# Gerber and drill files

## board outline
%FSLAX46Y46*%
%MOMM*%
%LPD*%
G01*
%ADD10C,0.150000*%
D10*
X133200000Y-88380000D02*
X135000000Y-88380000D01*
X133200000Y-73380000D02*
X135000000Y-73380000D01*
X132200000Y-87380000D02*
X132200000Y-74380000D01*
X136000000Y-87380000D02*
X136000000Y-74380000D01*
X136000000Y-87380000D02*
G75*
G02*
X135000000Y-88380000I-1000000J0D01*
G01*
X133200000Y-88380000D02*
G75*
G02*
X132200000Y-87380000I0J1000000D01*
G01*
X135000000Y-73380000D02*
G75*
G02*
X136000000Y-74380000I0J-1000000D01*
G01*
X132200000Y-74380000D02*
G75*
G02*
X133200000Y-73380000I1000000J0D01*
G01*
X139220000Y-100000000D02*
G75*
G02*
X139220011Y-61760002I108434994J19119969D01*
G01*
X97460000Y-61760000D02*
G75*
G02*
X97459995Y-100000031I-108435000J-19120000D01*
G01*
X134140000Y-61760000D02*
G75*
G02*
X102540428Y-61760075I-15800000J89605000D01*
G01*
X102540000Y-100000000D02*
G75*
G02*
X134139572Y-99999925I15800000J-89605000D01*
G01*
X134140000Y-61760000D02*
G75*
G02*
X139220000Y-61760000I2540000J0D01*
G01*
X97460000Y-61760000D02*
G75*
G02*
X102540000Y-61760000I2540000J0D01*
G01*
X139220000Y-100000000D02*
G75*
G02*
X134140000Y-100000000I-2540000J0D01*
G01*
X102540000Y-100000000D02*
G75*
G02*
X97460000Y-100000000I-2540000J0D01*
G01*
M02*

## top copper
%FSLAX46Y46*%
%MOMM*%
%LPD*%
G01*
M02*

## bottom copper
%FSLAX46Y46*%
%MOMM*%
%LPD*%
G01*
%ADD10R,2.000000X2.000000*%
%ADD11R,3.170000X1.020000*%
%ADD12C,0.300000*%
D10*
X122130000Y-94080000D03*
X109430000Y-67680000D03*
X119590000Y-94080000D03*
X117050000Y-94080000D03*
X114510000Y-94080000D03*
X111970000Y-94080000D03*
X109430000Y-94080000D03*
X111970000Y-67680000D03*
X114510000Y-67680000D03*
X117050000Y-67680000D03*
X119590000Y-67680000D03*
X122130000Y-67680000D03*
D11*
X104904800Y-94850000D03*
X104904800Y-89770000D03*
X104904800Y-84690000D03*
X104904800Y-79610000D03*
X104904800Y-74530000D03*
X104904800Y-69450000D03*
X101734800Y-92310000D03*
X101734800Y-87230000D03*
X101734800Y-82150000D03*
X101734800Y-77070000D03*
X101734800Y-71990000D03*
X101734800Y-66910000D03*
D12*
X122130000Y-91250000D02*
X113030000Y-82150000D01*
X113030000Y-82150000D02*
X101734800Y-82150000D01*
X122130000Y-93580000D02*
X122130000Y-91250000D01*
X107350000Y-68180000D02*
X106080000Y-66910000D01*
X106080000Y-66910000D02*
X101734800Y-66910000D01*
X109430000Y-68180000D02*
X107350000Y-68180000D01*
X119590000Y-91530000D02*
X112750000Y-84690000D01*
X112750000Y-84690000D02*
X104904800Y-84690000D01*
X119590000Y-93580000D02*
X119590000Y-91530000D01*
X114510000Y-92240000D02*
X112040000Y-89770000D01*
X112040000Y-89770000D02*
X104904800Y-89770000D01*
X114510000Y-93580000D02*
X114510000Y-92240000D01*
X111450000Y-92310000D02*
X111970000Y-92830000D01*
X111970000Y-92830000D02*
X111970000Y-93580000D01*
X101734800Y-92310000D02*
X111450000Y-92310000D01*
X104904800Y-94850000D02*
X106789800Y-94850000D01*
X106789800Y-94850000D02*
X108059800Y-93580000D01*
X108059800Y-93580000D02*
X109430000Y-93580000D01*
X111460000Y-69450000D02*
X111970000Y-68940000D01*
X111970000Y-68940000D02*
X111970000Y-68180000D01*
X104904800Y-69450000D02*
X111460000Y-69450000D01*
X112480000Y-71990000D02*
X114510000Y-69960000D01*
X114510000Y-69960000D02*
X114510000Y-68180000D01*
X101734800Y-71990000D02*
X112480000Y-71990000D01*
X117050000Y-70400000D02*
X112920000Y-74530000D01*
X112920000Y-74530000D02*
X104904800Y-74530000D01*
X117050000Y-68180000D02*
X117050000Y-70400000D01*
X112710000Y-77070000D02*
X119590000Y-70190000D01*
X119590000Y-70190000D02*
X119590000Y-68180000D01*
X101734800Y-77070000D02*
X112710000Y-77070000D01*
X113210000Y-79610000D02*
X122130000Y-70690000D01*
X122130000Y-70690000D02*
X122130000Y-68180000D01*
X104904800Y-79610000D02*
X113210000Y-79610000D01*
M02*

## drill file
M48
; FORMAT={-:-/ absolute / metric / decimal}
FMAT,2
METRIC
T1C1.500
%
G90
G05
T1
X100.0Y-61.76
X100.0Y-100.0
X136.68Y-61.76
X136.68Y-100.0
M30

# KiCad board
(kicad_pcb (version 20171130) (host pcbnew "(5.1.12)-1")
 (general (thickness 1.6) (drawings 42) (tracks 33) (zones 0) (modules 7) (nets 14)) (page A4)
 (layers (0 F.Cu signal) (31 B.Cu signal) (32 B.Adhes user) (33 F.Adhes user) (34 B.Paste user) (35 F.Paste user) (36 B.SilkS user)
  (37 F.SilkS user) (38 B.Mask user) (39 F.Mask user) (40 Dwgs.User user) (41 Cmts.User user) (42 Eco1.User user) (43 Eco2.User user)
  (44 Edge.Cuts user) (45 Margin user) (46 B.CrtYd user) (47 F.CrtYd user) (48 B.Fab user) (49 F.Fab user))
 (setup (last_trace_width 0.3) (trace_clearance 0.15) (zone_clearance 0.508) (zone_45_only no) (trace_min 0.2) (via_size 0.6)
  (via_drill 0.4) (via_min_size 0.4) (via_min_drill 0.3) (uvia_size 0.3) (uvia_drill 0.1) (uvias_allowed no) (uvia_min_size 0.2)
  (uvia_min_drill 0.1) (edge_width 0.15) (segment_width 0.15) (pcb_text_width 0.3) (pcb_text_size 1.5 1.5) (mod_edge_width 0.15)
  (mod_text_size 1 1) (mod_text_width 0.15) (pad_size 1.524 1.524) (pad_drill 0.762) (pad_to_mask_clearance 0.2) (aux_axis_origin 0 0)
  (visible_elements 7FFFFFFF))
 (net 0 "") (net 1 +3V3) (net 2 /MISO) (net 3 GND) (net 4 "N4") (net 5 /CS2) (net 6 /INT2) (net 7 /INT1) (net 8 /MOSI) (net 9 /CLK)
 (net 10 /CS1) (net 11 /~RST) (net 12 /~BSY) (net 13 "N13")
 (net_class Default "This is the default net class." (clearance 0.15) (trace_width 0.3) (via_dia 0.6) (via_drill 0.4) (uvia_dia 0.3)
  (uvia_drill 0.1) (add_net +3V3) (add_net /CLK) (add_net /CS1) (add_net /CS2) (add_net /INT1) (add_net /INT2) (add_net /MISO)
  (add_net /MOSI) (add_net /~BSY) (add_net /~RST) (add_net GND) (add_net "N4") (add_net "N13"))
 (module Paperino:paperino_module (layer B.Cu) (at 118.73 80.88 90)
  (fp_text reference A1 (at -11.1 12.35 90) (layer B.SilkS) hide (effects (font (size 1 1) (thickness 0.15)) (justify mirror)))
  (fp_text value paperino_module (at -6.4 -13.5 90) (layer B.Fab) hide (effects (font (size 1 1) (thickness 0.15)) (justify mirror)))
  (pad 1 smd rect (at -12.7 3.4 90) (size 2 2) (drill (offset -0.5 0)) (layers B.Cu B.Paste B.Mask) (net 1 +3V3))
  (pad 7 smd rect (at 12.7 -9.3 90) (size 2 2) (drill (offset 0.5 0)) (layers B.Cu B.Paste B.Mask) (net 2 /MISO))
  (pad 2 smd rect (at -12.7 0.86 90) (size 2 2) (drill (offset -0.5 0)) (layers B.Cu B.Paste B.Mask) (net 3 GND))
  (pad 3 smd rect (at -12.7 -1.68 90) (size 2 2) (drill (offset -0.5 0)) (layers B.Cu B.Paste B.Mask) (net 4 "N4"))
  (pad 4 smd rect (at -12.7 -4.22 90) (size 2 2) (drill (offset -0.5 0)) (layers B.Cu B.Paste B.Mask) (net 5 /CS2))
  (pad 5 smd rect (at -12.7 -6.76 90) (size 2 2) (drill (offset -0.5 0)) (layers B.Cu B.Paste B.Mask) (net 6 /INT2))
  (pad 6 smd rect (at -12.7 -9.3 90) (size 2 2) (drill (offset -0.5 0)) (layers B.Cu B.Paste B.Mask) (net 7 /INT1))
  (pad 8 smd rect (at 12.7 -6.76 90) (size 2 2) (drill (offset 0.5 0)) (layers B.Cu B.Paste B.Mask) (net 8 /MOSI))
  (pad 9 smd rect (at 12.7 -4.22 90) (size 2 2) (drill (offset 0.5 0)) (layers B.Cu B.Paste B.Mask) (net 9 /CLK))
  (pad 10 smd rect (at 12.7 -1.68 90) (size 2 2) (drill (offset 0.5 0)) (layers B.Cu B.Paste B.Mask) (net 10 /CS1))
  (pad 11 smd rect (at 12.7 0.86 90) (size 2 2) (drill (offset 0.5 0)) (layers B.Cu B.Paste B.Mask) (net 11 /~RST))
  (pad 12 smd rect (at 12.7 3.4 90) (size 2 2) (drill (offset 0.5 0)) (layers B.Cu B.Paste B.Mask) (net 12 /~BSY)))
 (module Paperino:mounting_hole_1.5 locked (layer F.Cu) (at 100 100)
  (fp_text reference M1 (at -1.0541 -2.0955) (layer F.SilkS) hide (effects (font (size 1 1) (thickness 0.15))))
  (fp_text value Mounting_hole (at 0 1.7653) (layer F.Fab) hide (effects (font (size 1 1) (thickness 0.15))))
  (pad "" np_thru_hole circle (at 0 0) (size 1.5 1.5) (drill 1.5) (layers *.Cu *.Mask)))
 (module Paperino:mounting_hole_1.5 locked (layer F.Cu) (at 136.68 100)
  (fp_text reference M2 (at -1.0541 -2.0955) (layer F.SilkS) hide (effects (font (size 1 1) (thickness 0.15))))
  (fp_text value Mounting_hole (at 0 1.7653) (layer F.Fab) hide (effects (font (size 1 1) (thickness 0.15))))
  (pad "" np_thru_hole circle (at 0 0) (size 1.5 1.5) (drill 1.5) (layers *.Cu *.Mask)))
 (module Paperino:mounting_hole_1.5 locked (layer F.Cu) (at 100 61.76)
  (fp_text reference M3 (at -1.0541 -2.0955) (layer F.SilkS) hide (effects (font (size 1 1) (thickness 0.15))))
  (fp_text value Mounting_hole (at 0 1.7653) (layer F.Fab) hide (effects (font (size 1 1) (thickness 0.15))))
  (pad "" np_thru_hole circle (at 0 0) (size 1.5 1.5) (drill 1.5) (layers *.Cu *.Mask)))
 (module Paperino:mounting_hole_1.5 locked (layer F.Cu) (at 136.68 61.76)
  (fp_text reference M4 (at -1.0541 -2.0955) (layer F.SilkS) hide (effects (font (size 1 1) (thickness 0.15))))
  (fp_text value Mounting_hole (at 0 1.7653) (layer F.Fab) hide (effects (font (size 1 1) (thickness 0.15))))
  (pad "" np_thru_hole circle (at 0 0) (size 1.5 1.5) (drill 1.5) (layers *.Cu *.Mask)))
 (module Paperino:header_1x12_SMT (layer B.Cu) (at 103.32 80.88 90)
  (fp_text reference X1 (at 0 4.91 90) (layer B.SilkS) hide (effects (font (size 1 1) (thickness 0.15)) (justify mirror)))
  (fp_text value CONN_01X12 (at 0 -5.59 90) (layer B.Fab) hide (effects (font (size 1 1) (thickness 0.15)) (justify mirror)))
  (pad 1 smd rect (at -13.97 1.5848 90) (size 1.02 3.17) (layers B.Cu B.Paste B.Mask) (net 7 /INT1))
  (pad 3 smd rect (at -8.89 1.5848 90) (size 1.02 3.17) (layers B.Cu B.Paste B.Mask) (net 5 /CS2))
  (pad 5 smd rect (at -3.81 1.5848 90) (size 1.02 3.17) (layers B.Cu B.Paste B.Mask) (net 3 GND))
  (pad 7 smd rect (at 1.27 1.5848 90) (size 1.02 3.17) (layers B.Cu B.Paste B.Mask) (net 12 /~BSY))
  (pad 9 smd rect (at 6.35 1.5848 90) (size 1.02 3.17) (layers B.Cu B.Paste B.Mask) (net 10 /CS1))
  (pad 11 smd rect (at 11.43 1.5848 90) (size 1.02 3.17) (layers B.Cu B.Paste B.Mask) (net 8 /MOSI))
  (pad 2 smd rect (at -11.43 -1.5852 90) (size 1.02 3.17) (layers B.Cu B.Paste B.Mask) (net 6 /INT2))
  (pad 4 smd rect (at -6.35 -1.5852 90) (size 1.02 3.17) (layers B.Cu B.Paste B.Mask) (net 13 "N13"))
  (pad 6 smd rect (at -1.27 -1.5852 90) (size 1.02 3.17) (layers B.Cu B.Paste B.Mask) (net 1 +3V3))
  (pad 8 smd rect (at 3.81 -1.5852 90) (size 1.02 3.17) (layers B.Cu B.Paste B.Mask) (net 11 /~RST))
  (pad 10 smd rect (at 8.89 -1.5852 90) (size 1.02 3.17) (layers B.Cu B.Paste B.Mask) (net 9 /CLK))
  (pad 12 smd rect (at 13.97 -1.5852 90) (size 1.02 3.17) (layers B.Cu B.Paste B.Mask) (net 2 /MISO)))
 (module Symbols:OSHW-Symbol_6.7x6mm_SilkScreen (layer F.Cu) (at 133.66 67.9 90)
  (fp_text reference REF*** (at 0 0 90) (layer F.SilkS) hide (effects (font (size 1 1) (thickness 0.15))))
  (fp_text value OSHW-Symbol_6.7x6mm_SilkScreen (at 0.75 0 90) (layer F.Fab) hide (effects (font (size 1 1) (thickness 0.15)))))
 (gr_line (start 133.2 88.38) (end 135 88.38) (layer Edge.Cuts) (width 0.15))
 (gr_line (start 133.2 73.38) (end 135 73.38) (layer Edge.Cuts) (width 0.15))
 (gr_line (start 132.2 87.38) (end 132.2 74.38) (layer Edge.Cuts) (width 0.15))
 (gr_line (start 136 87.38) (end 136 74.38) (layer Edge.Cuts) (width 0.15))
 (gr_arc (start 135 87.38) (end 136 87.38) (angle 90) (layer Edge.Cuts) (width 0.15))
 (gr_arc (start 133.2 87.38) (end 133.2 88.38) (angle 90) (layer Edge.Cuts) (width 0.15))
 (gr_arc (start 135 74.38) (end 135 73.38) (angle 90) (layer Edge.Cuts) (width 0.15))
 (gr_arc (start 133.2 74.38) (end 132.2 74.38) (angle 90) (layer Edge.Cuts) (width 0.15))
 (gr_arc (start 247.654994 80.880031) (end 139.22 100) (angle 19.9999845) (layer Edge.Cuts) (width 0.15))
 (gr_arc (start -10.975 80.88) (end 97.46 61.76) (angle 20) (layer Edge.Cuts) (width 0.15))
 (gr_arc (start 118.34 -27.845) (end 134.14 61.76) (angle 20) (layer Edge.Cuts) (width 0.15))
 (gr_arc (start 118.34 189.605) (end 102.54 100) (angle 20) (layer Edge.Cuts) (width 0.15))
 (gr_arc (start 136.68 61.76) (end 134.14 61.76) (angle 180) (layer Edge.Cuts) (width 0.15))
 (gr_arc (start 100 61.76) (end 97.46 61.76) (angle 180) (layer Edge.Cuts) (width 0.15))
 (gr_arc (start 136.68 100) (end 139.22 100) (angle 180) (layer Edge.Cuts) (width 0.15))
 (gr_arc (start 100 100) (end 102.54 100) (angle 180) (layer Edge.Cuts) (width 0.15))
 (segment (start 122.13 91.25) (end 113.03 82.15) (width 0.3) (layer B.Cu) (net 1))
 (segment (start 113.03 82.15) (end 101.7348 82.15) (width 0.3) (layer B.Cu) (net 1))
 (segment (start 122.13 93.58) (end 122.13 91.25) (width 0.3) (layer B.Cu) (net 1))
 (segment (start 107.35 68.18) (end 106.08 66.91) (width 0.3) (layer B.Cu) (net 2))
 (segment (start 106.08 66.91) (end 101.7348 66.91) (width 0.3) (layer B.Cu) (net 2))
 (segment (start 109.43 68.18) (end 107.35 68.18) (width 0.3) (layer B.Cu) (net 2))
 (segment (start 119.59 91.53) (end 112.75 84.69) (width 0.3) (layer B.Cu) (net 3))
 (segment (start 112.75 84.69) (end 104.9048 84.69) (width 0.3) (layer B.Cu) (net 3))
 (segment (start 119.59 93.58) (end 119.59 91.53) (width 0.3) (layer B.Cu) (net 3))
 (segment (start 114.51 92.24) (end 112.04 89.77) (width 0.3) (layer B.Cu) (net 5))
 (segment (start 112.04 89.77) (end 104.9048 89.77) (width 0.3) (layer B.Cu) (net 5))
 (segment (start 114.51 93.58) (end 114.51 92.24) (width 0.3) (layer B.Cu) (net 5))
 (segment (start 111.45 92.31) (end 111.97 92.83) (width 0.3) (layer B.Cu) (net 6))
 (segment (start 111.97 92.83) (end 111.97 93.58) (width 0.3) (layer B.Cu) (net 6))
 (segment (start 101.7348 92.31) (end 111.45 92.31) (width 0.3) (layer B.Cu) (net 6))
 (segment (start 104.9048 94.85) (end 106.7898 94.85) (width 0.3) (layer B.Cu) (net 7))
 (segment (start 106.7898 94.85) (end 108.0598 93.58) (width 0.3) (layer B.Cu) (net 7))
 (segment (start 108.0598 93.58) (end 109.43 93.58) (width 0.3) (layer B.Cu) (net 7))
 (segment (start 111.46 69.45) (end 111.97 68.94) (width 0.3) (layer B.Cu) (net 8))
 (segment (start 111.97 68.94) (end 111.97 68.18) (width 0.3) (layer B.Cu) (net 8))
 (segment (start 104.9048 69.45) (end 111.46 69.45) (width 0.3) (layer B.Cu) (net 8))
 (segment (start 112.48 71.99) (end 114.51 69.96) (width 0.3) (layer B.Cu) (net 9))
 (segment (start 114.51 69.96) (end 114.51 68.18) (width 0.3) (layer B.Cu) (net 9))
 (segment (start 101.7348 71.99) (end 112.48 71.99) (width 0.3) (layer B.Cu) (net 9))
 (segment (start 117.05 70.4) (end 112.92 74.53) (width 0.3) (layer B.Cu) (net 10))
 (segment (start 112.92 74.53) (end 104.9048 74.53) (width 0.3) (layer B.Cu) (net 10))
 (segment (start 117.05 68.18) (end 117.05 70.4) (width 0.3) (layer B.Cu) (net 10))
 (segment (start 112.71 77.07) (end 119.59 70.19) (width 0.3) (layer B.Cu) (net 11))
 (segment (start 119.59 70.19) (end 119.59 68.18) (width 0.3) (layer B.Cu) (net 11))
 (segment (start 101.7348 77.07) (end 112.71 77.07) (width 0.3) (layer B.Cu) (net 11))
 (segment (start 113.21 79.61) (end 122.13 70.69) (width 0.3) (layer B.Cu) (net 12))
 (segment (start 122.13 70.69) (end 122.13 68.18) (width 0.3) (layer B.Cu) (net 12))
 (segment (start 104.9048 79.61) (end 113.21 79.61) (width 0.3) (layer B.Cu) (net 12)))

